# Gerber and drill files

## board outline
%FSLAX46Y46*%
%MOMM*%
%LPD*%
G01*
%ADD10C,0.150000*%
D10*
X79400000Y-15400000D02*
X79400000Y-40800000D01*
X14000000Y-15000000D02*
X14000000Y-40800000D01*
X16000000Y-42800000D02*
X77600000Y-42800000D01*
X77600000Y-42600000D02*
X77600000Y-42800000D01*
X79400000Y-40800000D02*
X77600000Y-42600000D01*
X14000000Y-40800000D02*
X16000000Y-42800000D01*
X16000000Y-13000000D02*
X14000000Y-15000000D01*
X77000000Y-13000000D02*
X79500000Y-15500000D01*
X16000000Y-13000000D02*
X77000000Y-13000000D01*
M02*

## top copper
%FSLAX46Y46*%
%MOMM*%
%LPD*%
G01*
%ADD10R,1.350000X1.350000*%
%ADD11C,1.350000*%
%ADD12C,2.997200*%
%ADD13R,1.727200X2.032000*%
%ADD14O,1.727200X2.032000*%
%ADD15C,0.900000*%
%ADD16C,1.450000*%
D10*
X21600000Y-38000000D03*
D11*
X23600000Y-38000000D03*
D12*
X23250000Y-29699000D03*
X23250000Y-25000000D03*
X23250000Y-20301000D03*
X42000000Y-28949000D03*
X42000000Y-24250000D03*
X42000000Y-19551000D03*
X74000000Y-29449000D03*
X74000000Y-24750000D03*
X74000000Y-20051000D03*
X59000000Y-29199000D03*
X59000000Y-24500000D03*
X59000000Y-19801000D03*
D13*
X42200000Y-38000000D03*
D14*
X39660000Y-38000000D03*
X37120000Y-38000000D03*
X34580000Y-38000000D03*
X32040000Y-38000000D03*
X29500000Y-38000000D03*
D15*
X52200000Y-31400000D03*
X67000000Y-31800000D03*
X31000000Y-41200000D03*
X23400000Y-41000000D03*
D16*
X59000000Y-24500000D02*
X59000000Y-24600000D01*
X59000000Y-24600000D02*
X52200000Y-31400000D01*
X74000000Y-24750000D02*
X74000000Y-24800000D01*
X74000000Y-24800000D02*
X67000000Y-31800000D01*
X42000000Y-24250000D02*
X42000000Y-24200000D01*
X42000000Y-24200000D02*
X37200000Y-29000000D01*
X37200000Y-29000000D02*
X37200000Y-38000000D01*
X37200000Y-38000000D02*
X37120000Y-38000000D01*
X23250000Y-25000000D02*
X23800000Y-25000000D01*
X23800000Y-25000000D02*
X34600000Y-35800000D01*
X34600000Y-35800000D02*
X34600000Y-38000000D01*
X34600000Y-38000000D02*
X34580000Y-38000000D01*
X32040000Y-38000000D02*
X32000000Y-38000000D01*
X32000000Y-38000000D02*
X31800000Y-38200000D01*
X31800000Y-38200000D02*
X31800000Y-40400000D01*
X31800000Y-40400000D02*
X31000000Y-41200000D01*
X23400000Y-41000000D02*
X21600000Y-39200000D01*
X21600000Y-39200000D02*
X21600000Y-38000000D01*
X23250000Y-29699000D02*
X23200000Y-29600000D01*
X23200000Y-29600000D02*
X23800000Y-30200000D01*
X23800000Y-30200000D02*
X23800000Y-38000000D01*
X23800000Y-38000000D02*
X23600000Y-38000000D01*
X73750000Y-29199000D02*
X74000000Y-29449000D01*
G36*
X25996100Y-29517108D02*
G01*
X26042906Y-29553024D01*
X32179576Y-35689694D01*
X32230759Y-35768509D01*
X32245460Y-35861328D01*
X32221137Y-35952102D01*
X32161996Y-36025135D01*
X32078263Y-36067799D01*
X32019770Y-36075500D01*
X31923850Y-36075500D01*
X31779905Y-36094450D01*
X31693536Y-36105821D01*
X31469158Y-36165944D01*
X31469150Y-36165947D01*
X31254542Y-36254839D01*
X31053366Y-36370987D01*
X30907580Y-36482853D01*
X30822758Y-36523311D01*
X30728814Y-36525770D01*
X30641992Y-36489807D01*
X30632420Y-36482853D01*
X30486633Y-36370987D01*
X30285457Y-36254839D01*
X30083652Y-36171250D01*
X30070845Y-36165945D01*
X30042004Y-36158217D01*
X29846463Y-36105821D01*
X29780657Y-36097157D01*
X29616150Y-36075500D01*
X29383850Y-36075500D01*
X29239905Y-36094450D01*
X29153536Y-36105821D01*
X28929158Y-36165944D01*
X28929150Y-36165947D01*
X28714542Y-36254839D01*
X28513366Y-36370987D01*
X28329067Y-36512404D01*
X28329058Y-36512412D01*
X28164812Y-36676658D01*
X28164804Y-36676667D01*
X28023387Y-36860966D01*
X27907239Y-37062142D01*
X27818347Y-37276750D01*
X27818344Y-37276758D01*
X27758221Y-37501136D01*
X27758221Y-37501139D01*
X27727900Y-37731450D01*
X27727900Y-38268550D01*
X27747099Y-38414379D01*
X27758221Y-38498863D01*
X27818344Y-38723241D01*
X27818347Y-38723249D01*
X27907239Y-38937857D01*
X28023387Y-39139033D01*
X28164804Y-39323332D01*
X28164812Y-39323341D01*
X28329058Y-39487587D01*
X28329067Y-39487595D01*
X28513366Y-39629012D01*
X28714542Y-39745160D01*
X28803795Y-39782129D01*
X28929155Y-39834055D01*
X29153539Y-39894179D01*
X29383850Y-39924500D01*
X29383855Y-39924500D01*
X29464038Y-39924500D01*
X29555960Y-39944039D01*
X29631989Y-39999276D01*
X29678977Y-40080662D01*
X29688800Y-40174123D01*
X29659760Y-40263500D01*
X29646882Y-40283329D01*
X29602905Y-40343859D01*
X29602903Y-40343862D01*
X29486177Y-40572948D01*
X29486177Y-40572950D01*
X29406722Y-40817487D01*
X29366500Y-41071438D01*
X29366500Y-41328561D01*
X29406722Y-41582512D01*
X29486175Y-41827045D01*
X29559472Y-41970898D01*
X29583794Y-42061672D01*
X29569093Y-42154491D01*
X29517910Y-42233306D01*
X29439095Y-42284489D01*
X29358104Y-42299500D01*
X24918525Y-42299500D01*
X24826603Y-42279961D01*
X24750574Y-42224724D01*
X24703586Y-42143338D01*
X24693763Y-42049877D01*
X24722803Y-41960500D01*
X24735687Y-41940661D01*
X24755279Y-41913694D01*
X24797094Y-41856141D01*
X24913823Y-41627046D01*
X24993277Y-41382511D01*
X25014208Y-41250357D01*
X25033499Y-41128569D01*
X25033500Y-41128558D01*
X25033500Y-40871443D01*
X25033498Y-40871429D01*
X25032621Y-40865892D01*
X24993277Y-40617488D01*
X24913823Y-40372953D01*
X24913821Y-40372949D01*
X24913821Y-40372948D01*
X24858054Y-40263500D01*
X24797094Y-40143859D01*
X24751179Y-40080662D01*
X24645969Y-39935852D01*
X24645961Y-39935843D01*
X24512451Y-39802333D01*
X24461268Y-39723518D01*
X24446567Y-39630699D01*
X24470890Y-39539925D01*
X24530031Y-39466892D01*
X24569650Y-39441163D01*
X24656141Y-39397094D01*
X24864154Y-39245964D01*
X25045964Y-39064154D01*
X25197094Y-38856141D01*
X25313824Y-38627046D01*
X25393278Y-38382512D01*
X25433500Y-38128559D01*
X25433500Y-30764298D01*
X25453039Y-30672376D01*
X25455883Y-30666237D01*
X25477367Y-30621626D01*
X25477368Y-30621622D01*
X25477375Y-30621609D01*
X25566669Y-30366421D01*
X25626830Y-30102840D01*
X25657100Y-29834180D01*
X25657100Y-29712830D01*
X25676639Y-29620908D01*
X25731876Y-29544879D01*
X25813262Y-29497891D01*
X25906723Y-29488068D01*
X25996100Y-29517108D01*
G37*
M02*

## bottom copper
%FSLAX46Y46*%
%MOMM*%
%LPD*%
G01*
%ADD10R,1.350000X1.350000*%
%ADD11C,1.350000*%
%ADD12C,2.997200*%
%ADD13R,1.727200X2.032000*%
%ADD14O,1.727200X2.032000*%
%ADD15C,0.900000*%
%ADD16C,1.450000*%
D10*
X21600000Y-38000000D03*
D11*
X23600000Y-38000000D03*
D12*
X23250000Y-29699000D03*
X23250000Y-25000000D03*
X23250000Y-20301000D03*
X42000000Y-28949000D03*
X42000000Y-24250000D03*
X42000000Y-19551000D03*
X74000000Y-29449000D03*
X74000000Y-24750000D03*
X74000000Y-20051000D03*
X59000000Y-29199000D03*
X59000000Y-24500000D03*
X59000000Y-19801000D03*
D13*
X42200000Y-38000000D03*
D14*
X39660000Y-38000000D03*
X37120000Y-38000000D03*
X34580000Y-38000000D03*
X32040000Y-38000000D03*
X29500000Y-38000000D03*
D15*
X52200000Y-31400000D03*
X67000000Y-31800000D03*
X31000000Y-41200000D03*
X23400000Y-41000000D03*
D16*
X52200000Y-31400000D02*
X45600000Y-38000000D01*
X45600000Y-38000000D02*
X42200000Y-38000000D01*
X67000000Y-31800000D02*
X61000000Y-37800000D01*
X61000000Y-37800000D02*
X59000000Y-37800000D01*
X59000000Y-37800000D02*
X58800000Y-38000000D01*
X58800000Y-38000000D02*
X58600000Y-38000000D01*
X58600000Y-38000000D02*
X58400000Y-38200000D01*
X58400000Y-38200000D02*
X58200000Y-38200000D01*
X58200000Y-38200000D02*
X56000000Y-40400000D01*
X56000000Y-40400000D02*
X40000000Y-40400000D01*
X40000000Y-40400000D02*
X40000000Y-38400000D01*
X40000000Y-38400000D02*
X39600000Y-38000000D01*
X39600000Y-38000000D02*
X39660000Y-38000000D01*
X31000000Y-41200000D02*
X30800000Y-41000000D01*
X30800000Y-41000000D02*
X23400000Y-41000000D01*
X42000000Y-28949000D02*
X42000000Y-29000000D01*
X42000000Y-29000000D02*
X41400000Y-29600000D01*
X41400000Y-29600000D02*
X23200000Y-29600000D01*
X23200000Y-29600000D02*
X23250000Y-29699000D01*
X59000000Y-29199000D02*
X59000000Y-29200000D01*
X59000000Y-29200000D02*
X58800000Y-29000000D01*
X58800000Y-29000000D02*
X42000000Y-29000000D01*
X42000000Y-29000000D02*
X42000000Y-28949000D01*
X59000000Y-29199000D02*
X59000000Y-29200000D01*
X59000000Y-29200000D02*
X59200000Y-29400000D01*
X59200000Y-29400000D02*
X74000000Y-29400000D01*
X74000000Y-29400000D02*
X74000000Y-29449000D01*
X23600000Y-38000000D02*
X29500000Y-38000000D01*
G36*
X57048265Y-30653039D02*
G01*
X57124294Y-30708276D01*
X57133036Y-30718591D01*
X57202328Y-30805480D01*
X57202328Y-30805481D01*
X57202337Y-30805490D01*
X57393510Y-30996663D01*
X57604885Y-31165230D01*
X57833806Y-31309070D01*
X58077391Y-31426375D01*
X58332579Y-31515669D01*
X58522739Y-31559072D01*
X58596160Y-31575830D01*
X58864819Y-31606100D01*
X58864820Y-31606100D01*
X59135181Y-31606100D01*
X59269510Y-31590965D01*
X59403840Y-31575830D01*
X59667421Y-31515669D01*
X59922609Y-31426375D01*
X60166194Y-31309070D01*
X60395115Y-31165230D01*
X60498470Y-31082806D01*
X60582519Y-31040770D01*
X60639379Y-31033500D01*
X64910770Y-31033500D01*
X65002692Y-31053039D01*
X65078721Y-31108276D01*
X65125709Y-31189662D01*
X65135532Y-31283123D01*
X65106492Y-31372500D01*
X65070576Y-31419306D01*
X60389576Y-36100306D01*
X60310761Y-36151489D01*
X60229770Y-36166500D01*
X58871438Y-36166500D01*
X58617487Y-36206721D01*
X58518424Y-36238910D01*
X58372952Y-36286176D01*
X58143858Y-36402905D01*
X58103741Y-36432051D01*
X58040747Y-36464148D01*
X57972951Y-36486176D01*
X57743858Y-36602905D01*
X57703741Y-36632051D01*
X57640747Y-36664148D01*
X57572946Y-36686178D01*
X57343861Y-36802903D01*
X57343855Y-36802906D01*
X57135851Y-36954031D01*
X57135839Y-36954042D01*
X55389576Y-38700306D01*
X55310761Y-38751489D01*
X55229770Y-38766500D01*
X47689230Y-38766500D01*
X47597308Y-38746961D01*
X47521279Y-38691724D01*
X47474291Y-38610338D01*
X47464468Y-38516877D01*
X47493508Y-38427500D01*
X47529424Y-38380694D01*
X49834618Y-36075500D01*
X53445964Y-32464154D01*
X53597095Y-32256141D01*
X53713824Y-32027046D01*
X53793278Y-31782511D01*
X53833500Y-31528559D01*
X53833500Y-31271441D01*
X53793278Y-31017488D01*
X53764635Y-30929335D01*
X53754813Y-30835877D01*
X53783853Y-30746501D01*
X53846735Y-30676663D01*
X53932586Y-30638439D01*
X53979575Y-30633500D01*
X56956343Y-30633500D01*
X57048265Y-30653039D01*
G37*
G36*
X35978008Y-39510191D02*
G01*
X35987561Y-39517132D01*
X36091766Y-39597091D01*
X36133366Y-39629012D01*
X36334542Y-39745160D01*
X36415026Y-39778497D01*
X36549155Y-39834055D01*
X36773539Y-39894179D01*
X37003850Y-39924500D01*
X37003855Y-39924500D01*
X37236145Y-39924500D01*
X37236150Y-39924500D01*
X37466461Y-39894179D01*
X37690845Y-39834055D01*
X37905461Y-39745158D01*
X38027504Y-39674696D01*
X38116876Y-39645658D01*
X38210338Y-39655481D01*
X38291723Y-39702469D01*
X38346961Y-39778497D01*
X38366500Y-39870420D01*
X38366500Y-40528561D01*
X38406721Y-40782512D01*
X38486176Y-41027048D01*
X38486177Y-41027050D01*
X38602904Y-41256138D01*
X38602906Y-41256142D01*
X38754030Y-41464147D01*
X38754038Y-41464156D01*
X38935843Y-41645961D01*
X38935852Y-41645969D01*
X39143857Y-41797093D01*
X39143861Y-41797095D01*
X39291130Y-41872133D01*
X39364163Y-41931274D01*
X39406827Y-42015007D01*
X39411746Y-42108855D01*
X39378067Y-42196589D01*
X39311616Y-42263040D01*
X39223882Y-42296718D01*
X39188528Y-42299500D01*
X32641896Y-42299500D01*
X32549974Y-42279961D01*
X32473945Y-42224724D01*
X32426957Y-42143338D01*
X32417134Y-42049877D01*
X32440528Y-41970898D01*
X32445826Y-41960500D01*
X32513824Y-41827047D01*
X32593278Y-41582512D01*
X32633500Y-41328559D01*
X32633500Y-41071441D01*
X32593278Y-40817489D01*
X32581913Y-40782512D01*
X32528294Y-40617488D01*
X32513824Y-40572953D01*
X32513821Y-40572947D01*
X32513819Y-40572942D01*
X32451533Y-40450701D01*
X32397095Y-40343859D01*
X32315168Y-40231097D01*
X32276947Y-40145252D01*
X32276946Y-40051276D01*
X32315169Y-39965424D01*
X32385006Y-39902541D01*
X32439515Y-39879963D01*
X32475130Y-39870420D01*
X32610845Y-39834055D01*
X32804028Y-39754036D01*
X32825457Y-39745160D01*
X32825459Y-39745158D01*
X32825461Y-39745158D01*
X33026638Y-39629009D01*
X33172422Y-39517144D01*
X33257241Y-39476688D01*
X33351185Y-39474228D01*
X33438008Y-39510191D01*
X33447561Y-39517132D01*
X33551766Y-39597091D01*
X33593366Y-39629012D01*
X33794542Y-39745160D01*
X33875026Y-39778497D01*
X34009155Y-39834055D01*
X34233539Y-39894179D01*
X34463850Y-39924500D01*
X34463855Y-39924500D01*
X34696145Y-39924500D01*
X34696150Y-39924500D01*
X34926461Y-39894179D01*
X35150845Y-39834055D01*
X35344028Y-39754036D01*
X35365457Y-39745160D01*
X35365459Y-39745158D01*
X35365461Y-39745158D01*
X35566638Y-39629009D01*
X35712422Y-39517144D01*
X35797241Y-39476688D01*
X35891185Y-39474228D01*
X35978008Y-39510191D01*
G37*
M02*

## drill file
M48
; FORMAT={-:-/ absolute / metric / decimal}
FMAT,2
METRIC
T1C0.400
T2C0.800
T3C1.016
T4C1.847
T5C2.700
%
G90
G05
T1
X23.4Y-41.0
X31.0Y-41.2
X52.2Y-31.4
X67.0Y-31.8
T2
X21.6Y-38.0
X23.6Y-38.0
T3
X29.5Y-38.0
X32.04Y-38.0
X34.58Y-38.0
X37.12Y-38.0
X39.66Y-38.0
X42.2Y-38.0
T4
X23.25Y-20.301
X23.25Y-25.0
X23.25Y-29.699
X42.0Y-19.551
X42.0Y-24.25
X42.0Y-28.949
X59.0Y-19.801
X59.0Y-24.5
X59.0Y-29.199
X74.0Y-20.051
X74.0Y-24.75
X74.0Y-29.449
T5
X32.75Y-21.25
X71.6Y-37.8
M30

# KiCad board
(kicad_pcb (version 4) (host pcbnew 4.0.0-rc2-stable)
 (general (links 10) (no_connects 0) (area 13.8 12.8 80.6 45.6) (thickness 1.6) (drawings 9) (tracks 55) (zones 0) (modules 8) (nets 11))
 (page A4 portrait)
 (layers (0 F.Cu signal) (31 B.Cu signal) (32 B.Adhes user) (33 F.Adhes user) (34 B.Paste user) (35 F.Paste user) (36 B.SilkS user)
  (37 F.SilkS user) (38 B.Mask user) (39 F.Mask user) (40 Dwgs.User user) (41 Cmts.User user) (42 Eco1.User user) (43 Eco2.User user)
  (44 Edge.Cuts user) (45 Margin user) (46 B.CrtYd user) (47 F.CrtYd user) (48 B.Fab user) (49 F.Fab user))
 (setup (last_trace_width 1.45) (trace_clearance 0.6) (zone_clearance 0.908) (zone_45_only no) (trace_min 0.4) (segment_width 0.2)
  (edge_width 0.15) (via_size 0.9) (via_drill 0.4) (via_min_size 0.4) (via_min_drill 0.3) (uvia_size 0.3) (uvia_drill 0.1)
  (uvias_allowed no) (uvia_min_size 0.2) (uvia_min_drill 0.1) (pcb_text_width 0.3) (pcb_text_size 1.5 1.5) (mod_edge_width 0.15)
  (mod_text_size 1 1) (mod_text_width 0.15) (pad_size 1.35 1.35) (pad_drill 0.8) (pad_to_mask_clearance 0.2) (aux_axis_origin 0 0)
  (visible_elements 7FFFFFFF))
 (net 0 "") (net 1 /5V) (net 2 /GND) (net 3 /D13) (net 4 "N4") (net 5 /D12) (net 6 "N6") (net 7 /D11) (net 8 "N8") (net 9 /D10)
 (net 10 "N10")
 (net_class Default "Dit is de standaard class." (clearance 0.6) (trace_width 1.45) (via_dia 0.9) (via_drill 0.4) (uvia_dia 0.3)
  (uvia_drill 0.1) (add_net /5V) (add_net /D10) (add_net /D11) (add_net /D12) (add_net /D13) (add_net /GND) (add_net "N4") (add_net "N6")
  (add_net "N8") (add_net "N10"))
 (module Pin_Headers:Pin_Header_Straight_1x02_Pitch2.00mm (layer F.Cu) (at 21.6 38 90)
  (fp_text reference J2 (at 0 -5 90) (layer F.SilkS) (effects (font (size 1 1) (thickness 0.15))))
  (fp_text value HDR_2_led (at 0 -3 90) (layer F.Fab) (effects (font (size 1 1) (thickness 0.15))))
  (pad 1 thru_hole rect (at 0 0 90) (size 1.35 1.35) (drill 0.8) (layers *.Cu *.Mask) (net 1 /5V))
  (pad 2 thru_hole circle (at 0 2 90) (size 1.35 1.35) (drill 0.8) (layers *.Cu *.Mask) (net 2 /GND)))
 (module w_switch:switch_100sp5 (layer F.Cu) (at 23.25 25 90)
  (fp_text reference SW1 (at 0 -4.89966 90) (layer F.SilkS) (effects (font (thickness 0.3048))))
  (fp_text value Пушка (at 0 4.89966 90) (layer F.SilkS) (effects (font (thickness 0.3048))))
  (pad 1 thru_hole circle (at -4.699 0 90) (size 2.9972 2.9972) (drill 1.84658) (layers *.Cu *.Mask F.SilkS) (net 2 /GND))
  (pad 2 thru_hole circle (at 0 0 90) (size 2.9972 2.9972) (drill 1.84658) (layers *.Cu *.Mask F.SilkS) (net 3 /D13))
  (pad 3 thru_hole circle (at 4.699 0 90) (size 2.9972 2.9972) (drill 1.84658) (layers *.Cu *.Mask F.SilkS) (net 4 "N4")))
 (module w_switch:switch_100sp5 (layer F.Cu) (at 42 24.25 90)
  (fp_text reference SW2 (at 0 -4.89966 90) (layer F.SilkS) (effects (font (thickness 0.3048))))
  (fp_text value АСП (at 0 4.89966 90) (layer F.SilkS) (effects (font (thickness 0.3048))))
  (pad 1 thru_hole circle (at -4.699 0 90) (size 2.9972 2.9972) (drill 1.84658) (layers *.Cu *.Mask F.SilkS) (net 2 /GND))
  (pad 2 thru_hole circle (at 0 0 90) (size 2.9972 2.9972) (drill 1.84658) (layers *.Cu *.Mask F.SilkS) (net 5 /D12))
  (pad 3 thru_hole circle (at 4.699 0 90) (size 2.9972 2.9972) (drill 1.84658) (layers *.Cu *.Mask F.SilkS) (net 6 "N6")))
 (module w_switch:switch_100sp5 (layer F.Cu) (at 74 24.75 90)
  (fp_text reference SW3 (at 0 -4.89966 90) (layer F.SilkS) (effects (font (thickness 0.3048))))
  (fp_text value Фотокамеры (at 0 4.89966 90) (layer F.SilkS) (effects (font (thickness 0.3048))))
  (pad 1 thru_hole circle (at -4.699 0 90) (size 2.9972 2.9972) (drill 1.84658) (layers *.Cu *.Mask F.SilkS) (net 2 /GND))
  (pad 2 thru_hole circle (at 0 0 90) (size 2.9972 2.9972) (drill 1.84658) (layers *.Cu *.Mask F.SilkS) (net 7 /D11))
  (pad 3 thru_hole circle (at 4.699 0 90) (size 2.9972 2.9972) (drill 1.84658) (layers *.Cu *.Mask F.SilkS) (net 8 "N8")))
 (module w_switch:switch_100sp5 (layer F.Cu) (at 59 24.5 90)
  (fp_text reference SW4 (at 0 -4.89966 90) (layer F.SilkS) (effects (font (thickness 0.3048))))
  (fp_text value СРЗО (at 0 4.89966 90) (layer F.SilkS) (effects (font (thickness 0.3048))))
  (pad 1 thru_hole circle (at -4.699 0 90) (size 2.9972 2.9972) (drill 1.84658) (layers *.Cu *.Mask F.SilkS) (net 2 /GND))
  (pad 2 thru_hole circle (at 0 0 90) (size 2.9972 2.9972) (drill 1.84658) (layers *.Cu *.Mask F.SilkS) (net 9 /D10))
  (pad 3 thru_hole circle (at 4.699 0 90) (size 2.9972 2.9972) (drill 1.84658) (layers *.Cu *.Mask F.SilkS) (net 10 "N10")))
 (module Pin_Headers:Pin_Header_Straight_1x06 (layer F.Cu) (at 42.2 38 270)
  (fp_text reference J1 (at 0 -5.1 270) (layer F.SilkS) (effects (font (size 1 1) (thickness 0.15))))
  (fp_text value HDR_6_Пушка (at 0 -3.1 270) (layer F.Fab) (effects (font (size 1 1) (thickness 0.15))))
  (pad 1 thru_hole rect (at 0 0 270) (size 2.032 1.7272) (drill 1.016) (layers *.Cu *.Mask F.SilkS) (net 9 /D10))
  (pad 2 thru_hole oval (at 0 2.54 270) (size 2.032 1.7272) (drill 1.016) (layers *.Cu *.Mask F.SilkS) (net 7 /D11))
  (pad 3 thru_hole oval (at 0 5.08 270) (size 2.032 1.7272) (drill 1.016) (layers *.Cu *.Mask F.SilkS) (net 5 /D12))
  (pad 4 thru_hole oval (at 0 7.62 270) (size 2.032 1.7272) (drill 1.016) (layers *.Cu *.Mask F.SilkS) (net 3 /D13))
  (pad 5 thru_hole oval (at 0 10.16 270) (size 2.032 1.7272) (drill 1.016) (layers *.Cu *.Mask F.SilkS) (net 1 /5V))
  (pad 6 thru_hole oval (at 0 12.7 270) (size 2.032 1.7272) (drill 1.016) (layers *.Cu *.Mask F.SilkS) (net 2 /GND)))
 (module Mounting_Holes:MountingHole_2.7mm (layer F.Cu) (at 32.75 21.25)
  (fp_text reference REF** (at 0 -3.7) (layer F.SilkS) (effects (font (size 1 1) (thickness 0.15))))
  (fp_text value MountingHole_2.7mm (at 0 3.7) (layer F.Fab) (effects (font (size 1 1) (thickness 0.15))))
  (pad 1 np_thru_hole circle (at 0 0) (size 2.7 2.7) (drill 2.7) (layers *.Cu *.Mask F.SilkS)))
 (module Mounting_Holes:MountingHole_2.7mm (layer F.Cu) (at 71.6 37.8)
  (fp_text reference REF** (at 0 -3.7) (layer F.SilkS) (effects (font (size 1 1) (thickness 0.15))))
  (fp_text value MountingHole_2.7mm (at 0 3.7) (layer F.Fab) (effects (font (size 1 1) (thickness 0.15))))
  (pad 1 np_thru_hole circle (at 0 0) (size 2.7 2.7) (drill 2.7) (layers *.Cu *.Mask F.SilkS)))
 (gr_line (start 79.4 15.4) (end 79.4 40.8) (angle 90) (layer Edge.Cuts) (width 0.15))
 (gr_line (start 14 15) (end 14 40.8) (angle 90) (layer Edge.Cuts) (width 0.15))
 (gr_line (start 16 42.8) (end 77.6 42.8) (angle 90) (layer Edge.Cuts) (width 0.15))
 (gr_line (start 77.6 42.6) (end 77.6 42.8) (angle 90) (layer Edge.Cuts) (width 0.15))
 (gr_line (start 79.4 40.8) (end 77.6 42.6) (angle 90) (layer Edge.Cuts) (width 0.15))
 (gr_line (start 14 40.8) (end 16 42.8) (angle 90) (layer Edge.Cuts) (width 0.15))
 (gr_line (start 16 13) (end 14 15) (angle 90) (layer Edge.Cuts) (width 0.15))
 (gr_line (start 77 13) (end 79.5 15.5) (angle 90) (layer Edge.Cuts) (width 0.15))
 (gr_line (start 16 13) (end 77 13) (angle 90) (layer Edge.Cuts) (width 0.15))
 (segment (start 59 24.5) (end 59 24.6) (width 1.45) (layer F.Cu) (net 9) (status 80000))
 (segment (start 59 24.6) (end 52.2 31.4) (width 1.45) (layer F.Cu) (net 9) (status 80000))
 (via (at 52.2 31.4) (size 0.9) (layers F.Cu B.Cu) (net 9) (status 80000))
 (segment (start 52.2 31.4) (end 45.6 38) (width 1.45) (layer B.Cu) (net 9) (status 80000))
 (segment (start 45.6 38) (end 42.2 38) (width 1.45) (layer B.Cu) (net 9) (status 80000))
 (segment (start 74 24.75) (end 74 24.8) (width 1.45) (layer F.Cu) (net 7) (status 80000))
 (segment (start 74 24.8) (end 67 31.8) (width 1.45) (layer F.Cu) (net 7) (status 80000))
 (via (at 67 31.8) (size 0.9) (layers F.Cu B.Cu) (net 7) (status 80000))
 (segment (start 67 31.8) (end 61 37.8) (width 1.45) (layer B.Cu) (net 7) (status 80000))
 (segment (start 61 37.8) (end 59 37.8) (width 1.45) (layer B.Cu) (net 7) (status 80000))
 (segment (start 59 37.8) (end 58.8 38) (width 1.45) (layer B.Cu) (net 7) (status 80000))
 (segment (start 58.8 38) (end 58.6 38) (width 1.45) (layer B.Cu) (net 7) (status 80000))
 (segment (start 58.6 38) (end 58.4 38.2) (width 1.45) (layer B.Cu) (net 7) (status 80000))
 (segment (start 58.4 38.2) (end 58.2 38.2) (width 1.45) (layer B.Cu) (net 7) (status 80000))
 (segment (start 58.2 38.2) (end 56 40.4) (width 1.45) (layer B.Cu) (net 7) (status 80000))
 (segment (start 56 40.4) (end 40 40.4) (width 1.45) (layer B.Cu) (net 7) (status 80000))
 (segment (start 40 40.4) (end 40 38.4) (width 1.45) (layer B.Cu) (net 7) (status 80000))
 (segment (start 40 38.4) (end 39.6 38) (width 1.45) (layer B.Cu) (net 7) (status 80000))
 (segment (start 39.6 38) (end 39.66 38) (width 1.45) (layer B.Cu) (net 7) (status 80000))
 (segment (start 42 24.25) (end 42 24.2) (width 1.45) (layer F.Cu) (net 5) (status 80000))
 (segment (start 42 24.2) (end 37.2 29) (width 1.45) (layer F.Cu) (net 5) (status 80000))
 (segment (start 37.2 29) (end 37.2 38) (width 1.45) (layer F.Cu) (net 5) (status 80000))
 (segment (start 37.2 38) (end 37.12 38) (width 1.45) (layer F.Cu) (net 5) (status 80000))
 (segment (start 23.25 25) (end 23.8 25) (width 1.45) (layer F.Cu) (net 3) (status 80000))
 (segment (start 23.8 25) (end 34.6 35.8) (width 1.45) (layer F.Cu) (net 3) (status 80000))
 (segment (start 34.6 35.8) (end 34.6 38) (width 1.45) (layer F.Cu) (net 3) (status 80000))
 (segment (start 34.6 38) (end 34.58 38) (width 1.45) (layer F.Cu) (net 3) (status 80000))
 (segment (start 32.04 38) (end 32 38) (width 1.45) (layer F.Cu) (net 1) (status 80000))
 (segment (start 32 38) (end 31.8 38.2) (width 1.45) (layer F.Cu) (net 1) (status 80000))
 (segment (start 31.8 38.2) (end 31.8 40.4) (width 1.45) (layer F.Cu) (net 1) (status 80000))
 (segment (start 31.8 40.4) (end 31 41.2) (width 1.45) (layer F.Cu) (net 1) (status 80000))
 (via (at 31 41.2) (size 0.9) (layers F.Cu B.Cu) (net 1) (status 80000))
 (segment (start 31 41.2) (end 30.8 41) (width 1.45) (layer B.Cu) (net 1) (status 80000))
 (segment (start 30.8 41) (end 23.4 41) (width 1.45) (layer B.Cu) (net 1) (status 80000))
 (via (at 23.4 41) (size 0.9) (layers F.Cu B.Cu) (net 1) (status 80000))
 (segment (start 23.4 41) (end 21.6 39.2) (width 1.45) (layer F.Cu) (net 1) (status 80000))
 (segment (start 21.6 39.2) (end 21.6 38) (width 1.45) (layer F.Cu) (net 1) (status 80000))
 (segment (start 42 28.949) (end 42 29) (width 1.45) (layer B.Cu) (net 2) (status 80000))
 (segment (start 42 29) (end 41.4 29.6) (width 1.45) (layer B.Cu) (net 2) (status 80000))
 (segment (start 41.4 29.6) (end 23.2 29.6) (width 1.45) (layer B.Cu) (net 2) (status 80000))
 (segment (start 23.2 29.6) (end 23.25 29.699) (width 1.45) (layer B.Cu) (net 2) (status 80000))
 (segment (start 59 29.199) (end 59 29.2) (width 1.45) (layer B.Cu) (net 2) (status 80000))
 (segment (start 59 29.2) (end 58.8 29) (width 1.45) (layer B.Cu) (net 2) (status 80000))
 (segment (start 58.8 29) (end 42 29) (width 1.45) (layer B.Cu) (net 2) (status 80000))
 (segment (start 42 29) (end 42 28.949) (width 1.45) (layer B.Cu) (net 2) (status 80000))
 (segment (start 59 29.199) (end 59 29.2) (width 1.45) (layer B.Cu) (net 2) (status 80000))
 (segment (start 59 29.2) (end 59.2 29.4) (width 1.45) (layer B.Cu) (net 2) (status 80000))
 (segment (start 59.2 29.4) (end 74 29.4) (width 1.45) (layer B.Cu) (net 2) (status 80000))
 (segment (start 74 29.4) (end 74 29.449) (width 1.45) (layer B.Cu) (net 2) (status 80000))
 (segment (start 23.25 29.699) (end 23.2 29.6) (width 1.45) (layer F.Cu) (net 2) (status 80000))
 (segment (start 23.2 29.6) (end 23.8 30.2) (width 1.45) (layer F.Cu) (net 2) (status 80000))
 (segment (start 23.8 30.2) (end 23.8 38) (width 1.45) (layer F.Cu) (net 2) (status 80000))
 (segment (start 23.8 38) (end 23.6 38) (width 1.45) (layer F.Cu) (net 2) (status 80000))
 (segment (start 23.6 38) (end 29.5 38) (width 1.45) (layer B.Cu) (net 2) (status 80000))
 (segment (start 73.75 29.199) (end 74 29.449) (width 1.45) (layer F.Cu) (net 2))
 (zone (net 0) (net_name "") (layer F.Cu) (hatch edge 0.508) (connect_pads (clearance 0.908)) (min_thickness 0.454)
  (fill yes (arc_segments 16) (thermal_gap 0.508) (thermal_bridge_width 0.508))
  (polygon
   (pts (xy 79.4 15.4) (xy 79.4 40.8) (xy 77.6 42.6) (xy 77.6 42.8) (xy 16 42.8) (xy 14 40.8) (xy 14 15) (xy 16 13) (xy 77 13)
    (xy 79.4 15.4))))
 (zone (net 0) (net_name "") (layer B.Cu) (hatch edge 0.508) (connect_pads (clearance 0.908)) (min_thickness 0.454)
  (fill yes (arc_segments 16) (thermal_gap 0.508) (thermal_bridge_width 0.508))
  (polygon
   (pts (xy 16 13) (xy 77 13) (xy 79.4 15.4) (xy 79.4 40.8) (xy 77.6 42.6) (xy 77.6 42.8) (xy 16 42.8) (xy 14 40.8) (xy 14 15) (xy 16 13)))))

